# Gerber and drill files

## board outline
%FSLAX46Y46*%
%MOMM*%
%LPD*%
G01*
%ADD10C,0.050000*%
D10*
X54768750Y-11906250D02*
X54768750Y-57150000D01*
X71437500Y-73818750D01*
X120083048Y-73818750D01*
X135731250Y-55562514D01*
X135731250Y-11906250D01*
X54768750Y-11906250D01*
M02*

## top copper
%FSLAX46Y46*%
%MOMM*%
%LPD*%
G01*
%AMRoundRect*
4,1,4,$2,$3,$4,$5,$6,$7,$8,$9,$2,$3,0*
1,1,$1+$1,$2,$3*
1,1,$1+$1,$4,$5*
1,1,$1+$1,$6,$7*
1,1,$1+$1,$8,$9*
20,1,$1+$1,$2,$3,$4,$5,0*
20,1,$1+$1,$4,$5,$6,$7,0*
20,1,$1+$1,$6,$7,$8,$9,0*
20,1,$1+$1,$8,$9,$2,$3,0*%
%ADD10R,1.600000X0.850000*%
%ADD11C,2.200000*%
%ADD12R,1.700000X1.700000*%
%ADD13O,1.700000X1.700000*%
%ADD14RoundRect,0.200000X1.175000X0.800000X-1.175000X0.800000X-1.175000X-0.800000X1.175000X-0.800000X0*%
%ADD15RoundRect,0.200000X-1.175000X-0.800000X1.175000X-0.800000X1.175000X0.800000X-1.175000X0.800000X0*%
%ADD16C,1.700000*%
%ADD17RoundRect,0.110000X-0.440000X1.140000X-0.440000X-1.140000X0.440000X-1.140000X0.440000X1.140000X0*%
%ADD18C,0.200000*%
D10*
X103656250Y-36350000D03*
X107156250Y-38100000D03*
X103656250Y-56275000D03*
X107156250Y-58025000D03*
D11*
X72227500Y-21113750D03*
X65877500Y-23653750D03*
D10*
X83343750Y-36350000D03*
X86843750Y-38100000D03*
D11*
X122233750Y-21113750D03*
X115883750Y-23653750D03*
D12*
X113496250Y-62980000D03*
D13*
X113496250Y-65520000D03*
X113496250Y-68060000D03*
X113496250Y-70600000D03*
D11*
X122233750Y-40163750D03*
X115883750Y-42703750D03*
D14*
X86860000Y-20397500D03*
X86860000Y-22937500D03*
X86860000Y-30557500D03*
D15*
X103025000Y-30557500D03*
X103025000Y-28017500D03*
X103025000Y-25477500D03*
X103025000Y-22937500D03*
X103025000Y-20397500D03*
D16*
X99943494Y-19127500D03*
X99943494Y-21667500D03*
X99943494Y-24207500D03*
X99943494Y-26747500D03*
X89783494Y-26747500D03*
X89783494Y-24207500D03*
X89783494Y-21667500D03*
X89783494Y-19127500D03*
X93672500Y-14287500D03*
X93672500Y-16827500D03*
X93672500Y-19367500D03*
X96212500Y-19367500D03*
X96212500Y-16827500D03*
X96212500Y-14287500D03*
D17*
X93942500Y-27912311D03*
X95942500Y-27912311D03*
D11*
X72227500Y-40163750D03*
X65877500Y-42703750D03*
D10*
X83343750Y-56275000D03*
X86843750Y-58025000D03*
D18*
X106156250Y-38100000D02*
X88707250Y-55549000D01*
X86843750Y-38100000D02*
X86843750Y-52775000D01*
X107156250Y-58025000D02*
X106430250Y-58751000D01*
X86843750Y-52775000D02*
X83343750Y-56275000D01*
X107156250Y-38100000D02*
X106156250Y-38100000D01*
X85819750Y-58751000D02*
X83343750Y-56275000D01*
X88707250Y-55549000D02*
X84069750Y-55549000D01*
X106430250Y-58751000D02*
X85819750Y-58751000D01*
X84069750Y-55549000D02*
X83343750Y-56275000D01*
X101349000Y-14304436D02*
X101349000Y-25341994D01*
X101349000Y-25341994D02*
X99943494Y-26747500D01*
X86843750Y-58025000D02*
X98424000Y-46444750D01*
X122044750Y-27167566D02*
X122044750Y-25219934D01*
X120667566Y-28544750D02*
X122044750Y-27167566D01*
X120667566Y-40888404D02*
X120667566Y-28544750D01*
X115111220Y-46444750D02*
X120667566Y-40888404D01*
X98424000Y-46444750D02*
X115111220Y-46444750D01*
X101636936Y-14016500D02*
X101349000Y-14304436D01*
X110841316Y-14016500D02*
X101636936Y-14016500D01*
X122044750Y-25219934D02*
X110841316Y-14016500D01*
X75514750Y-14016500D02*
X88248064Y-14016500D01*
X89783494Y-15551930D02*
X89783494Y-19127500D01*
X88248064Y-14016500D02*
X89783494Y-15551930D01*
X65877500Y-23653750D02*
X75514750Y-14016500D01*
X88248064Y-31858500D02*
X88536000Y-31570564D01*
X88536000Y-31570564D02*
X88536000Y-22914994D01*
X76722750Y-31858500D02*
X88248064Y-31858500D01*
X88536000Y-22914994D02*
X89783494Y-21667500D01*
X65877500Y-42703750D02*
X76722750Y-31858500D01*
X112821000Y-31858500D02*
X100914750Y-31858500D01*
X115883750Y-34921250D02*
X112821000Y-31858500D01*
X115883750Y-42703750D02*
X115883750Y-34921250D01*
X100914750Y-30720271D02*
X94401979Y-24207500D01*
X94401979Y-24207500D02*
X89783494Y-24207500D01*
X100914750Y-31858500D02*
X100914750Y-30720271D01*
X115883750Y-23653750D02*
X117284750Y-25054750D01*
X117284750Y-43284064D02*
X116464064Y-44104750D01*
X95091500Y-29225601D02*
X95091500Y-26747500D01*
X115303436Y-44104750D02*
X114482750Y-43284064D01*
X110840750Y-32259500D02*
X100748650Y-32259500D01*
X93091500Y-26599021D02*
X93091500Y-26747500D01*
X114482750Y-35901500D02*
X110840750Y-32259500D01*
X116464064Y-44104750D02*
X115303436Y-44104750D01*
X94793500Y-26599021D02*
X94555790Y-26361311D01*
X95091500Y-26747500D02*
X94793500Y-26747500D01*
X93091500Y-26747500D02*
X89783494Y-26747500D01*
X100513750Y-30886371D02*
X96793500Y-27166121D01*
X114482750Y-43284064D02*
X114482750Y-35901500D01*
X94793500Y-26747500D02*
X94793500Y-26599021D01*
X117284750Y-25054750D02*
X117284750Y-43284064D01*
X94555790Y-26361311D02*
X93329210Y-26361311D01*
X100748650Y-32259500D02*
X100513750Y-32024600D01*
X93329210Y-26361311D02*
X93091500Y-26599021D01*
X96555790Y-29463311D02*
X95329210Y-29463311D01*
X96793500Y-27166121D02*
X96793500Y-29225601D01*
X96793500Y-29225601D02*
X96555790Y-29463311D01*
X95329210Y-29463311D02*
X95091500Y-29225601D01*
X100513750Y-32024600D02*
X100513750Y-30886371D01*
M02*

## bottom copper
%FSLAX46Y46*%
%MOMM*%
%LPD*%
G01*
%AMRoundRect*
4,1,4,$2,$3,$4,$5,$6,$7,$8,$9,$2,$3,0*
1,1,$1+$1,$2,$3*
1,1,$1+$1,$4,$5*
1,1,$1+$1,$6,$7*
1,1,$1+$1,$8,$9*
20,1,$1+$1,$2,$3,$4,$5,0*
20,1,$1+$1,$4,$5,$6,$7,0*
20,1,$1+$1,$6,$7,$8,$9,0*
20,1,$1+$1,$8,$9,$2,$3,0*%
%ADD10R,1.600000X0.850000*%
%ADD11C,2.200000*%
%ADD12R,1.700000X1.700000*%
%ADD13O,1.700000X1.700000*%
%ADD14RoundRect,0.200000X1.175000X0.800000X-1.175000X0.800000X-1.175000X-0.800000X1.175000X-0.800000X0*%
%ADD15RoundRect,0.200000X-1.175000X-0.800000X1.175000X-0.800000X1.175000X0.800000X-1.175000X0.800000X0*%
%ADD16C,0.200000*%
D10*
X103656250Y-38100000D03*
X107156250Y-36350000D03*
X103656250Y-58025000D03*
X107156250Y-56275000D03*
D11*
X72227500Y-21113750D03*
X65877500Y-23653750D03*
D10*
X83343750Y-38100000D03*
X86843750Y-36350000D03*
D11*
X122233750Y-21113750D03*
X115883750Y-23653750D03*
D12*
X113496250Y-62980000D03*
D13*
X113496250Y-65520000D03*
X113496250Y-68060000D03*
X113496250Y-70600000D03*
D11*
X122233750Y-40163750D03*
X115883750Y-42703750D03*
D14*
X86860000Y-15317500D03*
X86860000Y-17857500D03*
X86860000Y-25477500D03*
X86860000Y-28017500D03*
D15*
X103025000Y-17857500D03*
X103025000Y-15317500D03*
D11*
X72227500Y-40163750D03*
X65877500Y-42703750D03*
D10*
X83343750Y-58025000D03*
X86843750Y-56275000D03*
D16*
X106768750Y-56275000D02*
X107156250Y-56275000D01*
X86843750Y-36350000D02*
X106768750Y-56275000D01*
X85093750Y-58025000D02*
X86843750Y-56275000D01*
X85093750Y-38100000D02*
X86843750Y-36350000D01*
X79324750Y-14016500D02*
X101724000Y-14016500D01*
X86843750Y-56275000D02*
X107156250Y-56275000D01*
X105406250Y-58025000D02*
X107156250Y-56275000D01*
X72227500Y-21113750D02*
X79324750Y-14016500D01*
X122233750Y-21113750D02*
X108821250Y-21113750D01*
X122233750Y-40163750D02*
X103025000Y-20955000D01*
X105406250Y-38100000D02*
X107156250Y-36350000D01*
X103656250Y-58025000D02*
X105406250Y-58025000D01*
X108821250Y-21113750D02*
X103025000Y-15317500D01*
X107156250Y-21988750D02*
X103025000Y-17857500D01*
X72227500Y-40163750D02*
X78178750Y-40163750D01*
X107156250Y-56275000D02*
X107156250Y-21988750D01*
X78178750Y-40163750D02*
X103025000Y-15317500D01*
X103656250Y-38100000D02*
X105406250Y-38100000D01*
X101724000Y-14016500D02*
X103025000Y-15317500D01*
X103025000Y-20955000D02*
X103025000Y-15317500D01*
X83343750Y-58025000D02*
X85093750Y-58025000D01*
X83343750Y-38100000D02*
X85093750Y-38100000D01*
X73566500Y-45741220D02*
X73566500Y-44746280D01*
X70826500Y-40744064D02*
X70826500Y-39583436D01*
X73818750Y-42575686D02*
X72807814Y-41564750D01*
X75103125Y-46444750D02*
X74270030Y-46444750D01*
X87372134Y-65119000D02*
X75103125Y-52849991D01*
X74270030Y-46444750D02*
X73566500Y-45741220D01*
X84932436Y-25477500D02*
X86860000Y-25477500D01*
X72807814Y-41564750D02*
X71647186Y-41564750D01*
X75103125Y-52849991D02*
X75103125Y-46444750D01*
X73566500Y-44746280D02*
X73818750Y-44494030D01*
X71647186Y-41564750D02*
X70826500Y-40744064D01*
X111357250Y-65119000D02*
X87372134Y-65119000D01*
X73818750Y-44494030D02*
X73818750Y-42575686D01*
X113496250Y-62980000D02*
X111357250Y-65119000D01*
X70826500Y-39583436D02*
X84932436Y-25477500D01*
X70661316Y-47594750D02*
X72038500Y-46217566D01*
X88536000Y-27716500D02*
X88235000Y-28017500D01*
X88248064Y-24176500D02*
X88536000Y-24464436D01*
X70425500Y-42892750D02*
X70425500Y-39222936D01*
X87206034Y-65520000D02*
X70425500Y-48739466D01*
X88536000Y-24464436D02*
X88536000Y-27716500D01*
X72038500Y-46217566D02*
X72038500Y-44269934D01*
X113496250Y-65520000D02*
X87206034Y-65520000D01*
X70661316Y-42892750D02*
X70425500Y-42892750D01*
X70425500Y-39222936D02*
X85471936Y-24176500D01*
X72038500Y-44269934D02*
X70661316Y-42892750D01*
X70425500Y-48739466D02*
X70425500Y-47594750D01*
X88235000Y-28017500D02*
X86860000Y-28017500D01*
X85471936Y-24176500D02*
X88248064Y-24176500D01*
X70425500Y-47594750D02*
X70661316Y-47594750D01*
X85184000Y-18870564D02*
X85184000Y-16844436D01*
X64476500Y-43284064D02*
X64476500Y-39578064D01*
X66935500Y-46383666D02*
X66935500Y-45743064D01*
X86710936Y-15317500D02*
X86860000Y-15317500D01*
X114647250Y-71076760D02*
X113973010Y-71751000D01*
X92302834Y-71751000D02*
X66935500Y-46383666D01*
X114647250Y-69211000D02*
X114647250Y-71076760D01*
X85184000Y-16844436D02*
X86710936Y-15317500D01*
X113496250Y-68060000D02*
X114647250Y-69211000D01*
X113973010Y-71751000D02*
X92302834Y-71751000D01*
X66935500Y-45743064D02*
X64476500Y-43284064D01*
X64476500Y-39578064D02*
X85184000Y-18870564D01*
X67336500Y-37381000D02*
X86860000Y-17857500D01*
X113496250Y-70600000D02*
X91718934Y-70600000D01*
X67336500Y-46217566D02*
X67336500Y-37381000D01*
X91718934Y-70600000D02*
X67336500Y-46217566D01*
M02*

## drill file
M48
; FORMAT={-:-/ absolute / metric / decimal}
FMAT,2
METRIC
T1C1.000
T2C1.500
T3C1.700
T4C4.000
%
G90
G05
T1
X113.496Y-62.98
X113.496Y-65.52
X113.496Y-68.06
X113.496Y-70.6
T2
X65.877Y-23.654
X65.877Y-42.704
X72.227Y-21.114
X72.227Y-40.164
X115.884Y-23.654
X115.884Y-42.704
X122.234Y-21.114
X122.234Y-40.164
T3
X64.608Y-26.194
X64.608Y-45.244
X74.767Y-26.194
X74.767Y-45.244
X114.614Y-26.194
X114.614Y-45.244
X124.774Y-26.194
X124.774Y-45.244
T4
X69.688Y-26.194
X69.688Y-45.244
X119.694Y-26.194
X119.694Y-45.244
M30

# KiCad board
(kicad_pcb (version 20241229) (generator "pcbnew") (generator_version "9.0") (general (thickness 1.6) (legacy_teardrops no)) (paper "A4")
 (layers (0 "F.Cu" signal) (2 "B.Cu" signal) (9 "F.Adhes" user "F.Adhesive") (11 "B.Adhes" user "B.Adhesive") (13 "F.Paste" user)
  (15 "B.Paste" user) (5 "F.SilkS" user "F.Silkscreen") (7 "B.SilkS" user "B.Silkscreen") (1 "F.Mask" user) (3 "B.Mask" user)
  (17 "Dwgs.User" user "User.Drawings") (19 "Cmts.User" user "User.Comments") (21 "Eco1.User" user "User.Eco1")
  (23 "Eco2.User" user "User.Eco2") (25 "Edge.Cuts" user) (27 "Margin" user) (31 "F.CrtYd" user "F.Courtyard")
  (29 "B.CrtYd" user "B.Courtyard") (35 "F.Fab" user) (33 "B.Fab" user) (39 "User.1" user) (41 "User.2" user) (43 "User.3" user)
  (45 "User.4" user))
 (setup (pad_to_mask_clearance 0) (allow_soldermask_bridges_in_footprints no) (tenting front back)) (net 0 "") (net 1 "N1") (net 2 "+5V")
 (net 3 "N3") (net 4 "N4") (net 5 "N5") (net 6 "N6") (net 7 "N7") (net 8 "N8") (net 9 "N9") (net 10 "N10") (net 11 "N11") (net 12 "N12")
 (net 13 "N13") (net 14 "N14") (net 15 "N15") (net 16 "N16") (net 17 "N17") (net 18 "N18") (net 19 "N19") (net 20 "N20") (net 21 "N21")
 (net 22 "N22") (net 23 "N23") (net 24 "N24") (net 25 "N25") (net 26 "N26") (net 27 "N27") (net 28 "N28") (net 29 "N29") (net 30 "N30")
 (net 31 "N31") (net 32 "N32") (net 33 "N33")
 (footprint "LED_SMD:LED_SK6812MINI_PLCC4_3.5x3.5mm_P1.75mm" (layer "F.Cu") (at 105.40625 37.225)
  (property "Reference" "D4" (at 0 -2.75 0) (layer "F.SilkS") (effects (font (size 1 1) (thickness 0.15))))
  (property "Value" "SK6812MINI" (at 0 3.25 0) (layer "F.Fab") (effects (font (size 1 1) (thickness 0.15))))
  (pad "1" smd rect (at -1.75 -0.875) (size 1.6 0.85) (layers "F.Cu" "F.Mask" "F.Paste") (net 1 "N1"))
  (pad "2" smd rect (at -1.75 0.875) (size 1.6 0.85) (layers "F.Mask" "B.Cu" "F.Paste") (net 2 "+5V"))
  (pad "3" smd rect (at 1.75 0.875) (size 1.6 0.85) (layers "F.Cu" "F.Mask" "F.Paste") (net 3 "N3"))
  (pad "4" smd rect (at 1.75 -0.875) (size 1.6 0.85) (layers "F.Mask" "B.Cu" "F.Paste") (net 2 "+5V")))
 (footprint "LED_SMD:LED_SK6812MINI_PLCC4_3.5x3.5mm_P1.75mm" (layer "F.Cu") (at 105.40625 57.15)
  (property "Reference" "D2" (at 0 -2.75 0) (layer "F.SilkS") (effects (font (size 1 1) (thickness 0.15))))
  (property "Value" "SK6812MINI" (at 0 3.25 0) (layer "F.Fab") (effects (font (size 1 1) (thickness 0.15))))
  (pad "1" smd rect (at -1.75 -0.875) (size 1.6 0.85) (layers "F.Cu" "F.Mask" "F.Paste") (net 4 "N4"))
  (pad "2" smd rect (at -1.75 0.875) (size 1.6 0.85) (layers "F.Mask" "B.Cu" "F.Paste") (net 2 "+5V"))
  (pad "3" smd rect (at 1.75 0.875) (size 1.6 0.85) (layers "F.Cu" "F.Mask" "F.Paste") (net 3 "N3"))
  (pad "4" smd rect (at 1.75 -0.875) (size 1.6 0.85) (layers "F.Mask" "B.Cu" "F.Paste") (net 2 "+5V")))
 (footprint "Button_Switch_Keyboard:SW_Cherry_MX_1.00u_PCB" (layer "F.Cu") (at 72.2275 21.11375)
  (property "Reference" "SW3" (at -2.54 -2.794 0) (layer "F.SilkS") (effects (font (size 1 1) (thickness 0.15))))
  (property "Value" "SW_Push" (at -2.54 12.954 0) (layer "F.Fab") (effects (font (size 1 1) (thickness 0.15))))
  (pad "" np_thru_hole circle (at -7.62 5.08) (size 1.7 1.7) (drill 1.7) (layers "*.Cu" "*.Mask"))
  (pad "" np_thru_hole circle (at -2.54 5.08) (size 4 4) (drill 4) (layers "*.Cu" "*.Mask"))
  (pad "" np_thru_hole circle (at 2.54 5.08) (size 1.7 1.7) (drill 1.7) (layers "*.Cu" "*.Mask"))
  (pad "1" thru_hole circle (at 0 0) (size 2.2 2.2) (drill 1.5) (layers "*.Cu" "*.Mask") (remove_unused_layers no) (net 2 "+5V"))
  (pad "2" thru_hole circle (at -6.35 2.54) (size 2.2 2.2) (drill 1.5) (layers "*.Cu" "*.Mask") (remove_unused_layers no) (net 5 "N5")))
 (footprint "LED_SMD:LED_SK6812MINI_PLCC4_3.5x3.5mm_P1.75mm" (layer "F.Cu") (at 85.09375 37.225)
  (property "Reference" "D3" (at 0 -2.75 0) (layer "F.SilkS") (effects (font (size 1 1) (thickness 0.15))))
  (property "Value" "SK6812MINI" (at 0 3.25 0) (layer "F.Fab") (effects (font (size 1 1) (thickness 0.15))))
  (pad "1" smd rect (at -1.75 -0.875) (size 1.6 0.85) (layers "F.Cu" "F.Mask" "F.Paste") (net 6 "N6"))
  (pad "2" smd rect (at -1.75 0.875) (size 1.6 0.85) (layers "F.Mask" "B.Cu" "F.Paste") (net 2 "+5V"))
  (pad "3" smd rect (at 1.75 0.875) (size 1.6 0.85) (layers "F.Cu" "F.Mask" "F.Paste") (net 3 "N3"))
  (pad "4" smd rect (at 1.75 -0.875) (size 1.6 0.85) (layers "F.Mask" "B.Cu" "F.Paste") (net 2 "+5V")))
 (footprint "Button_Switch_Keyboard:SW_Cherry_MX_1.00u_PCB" (layer "F.Cu") (at 122.23375 21.11375)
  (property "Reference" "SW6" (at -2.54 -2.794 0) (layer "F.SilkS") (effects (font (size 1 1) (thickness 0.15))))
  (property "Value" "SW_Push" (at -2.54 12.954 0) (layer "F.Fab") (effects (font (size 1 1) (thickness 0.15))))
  (pad "" np_thru_hole circle (at -7.62 5.08) (size 1.7 1.7) (drill 1.7) (layers "*.Cu" "*.Mask"))
  (pad "" np_thru_hole circle (at -2.54 5.08) (size 4 4) (drill 4) (layers "*.Cu" "*.Mask"))
  (pad "" np_thru_hole circle (at 2.54 5.08) (size 1.7 1.7) (drill 1.7) (layers "*.Cu" "*.Mask"))
  (pad "1" thru_hole circle (at 0 0) (size 2.2 2.2) (drill 1.5) (layers "*.Cu" "*.Mask") (remove_unused_layers no) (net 2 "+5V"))
  (pad "2" thru_hole circle (at -6.35 2.54) (size 2.2 2.2) (drill 1.5) (layers "*.Cu" "*.Mask") (remove_unused_layers no) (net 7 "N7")))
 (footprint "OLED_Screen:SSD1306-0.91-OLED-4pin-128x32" (layer "F.Cu") (at 76.99625 60.79)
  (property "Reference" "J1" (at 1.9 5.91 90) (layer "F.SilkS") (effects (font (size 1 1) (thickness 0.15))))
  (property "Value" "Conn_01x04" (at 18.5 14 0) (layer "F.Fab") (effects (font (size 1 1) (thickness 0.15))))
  (pad "1" thru_hole rect (at 36.5 2.19) (size 1.7 1.7) (drill 1) (layers "*.Cu" "*.Mask") (remove_unused_layers no) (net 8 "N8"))
  (pad "2" thru_hole oval (at 36.5 4.73) (size 1.7 1.7) (drill 1) (layers "*.Cu" "*.Mask") (remove_unused_layers no) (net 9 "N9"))
  (pad "3" thru_hole oval (at 36.5 7.27) (size 1.7 1.7) (drill 1) (layers "*.Cu" "*.Mask") (remove_unused_layers no) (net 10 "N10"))
  (pad "4" thru_hole oval (at 36.5 9.81) (size 1.7 1.7) (drill 1) (layers "*.Cu" "*.Mask") (remove_unused_layers no) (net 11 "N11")))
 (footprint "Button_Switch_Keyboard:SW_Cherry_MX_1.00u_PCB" (layer "F.Cu") (at 122.23375 40.16375)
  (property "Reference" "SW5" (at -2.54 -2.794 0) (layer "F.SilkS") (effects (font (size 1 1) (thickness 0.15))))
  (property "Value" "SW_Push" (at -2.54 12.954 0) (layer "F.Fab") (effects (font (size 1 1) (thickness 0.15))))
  (pad "" np_thru_hole circle (at -7.62 5.08) (size 1.7 1.7) (drill 1.7) (layers "*.Cu" "*.Mask"))
  (pad "" np_thru_hole circle (at -2.54 5.08) (size 4 4) (drill 4) (layers "*.Cu" "*.Mask"))
  (pad "" np_thru_hole circle (at 2.54 5.08) (size 1.7 1.7) (drill 1.7) (layers "*.Cu" "*.Mask"))
  (pad "1" thru_hole circle (at 0 0) (size 2.2 2.2) (drill 1.5) (layers "*.Cu" "*.Mask") (remove_unused_layers no) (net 2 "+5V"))
  (pad "2" thru_hole circle (at -6.35 2.54) (size 2.2 2.2) (drill 1.5) (layers "*.Cu" "*.Mask") (remove_unused_layers no) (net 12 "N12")))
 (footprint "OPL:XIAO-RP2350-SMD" (layer "F.Cu") (at 94.86 22.9375)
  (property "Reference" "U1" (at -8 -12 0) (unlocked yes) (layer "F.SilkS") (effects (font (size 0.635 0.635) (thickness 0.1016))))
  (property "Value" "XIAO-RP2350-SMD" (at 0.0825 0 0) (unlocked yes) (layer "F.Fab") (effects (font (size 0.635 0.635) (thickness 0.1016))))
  (pad "1" smd roundrect (at -8 -7.62 180) (size 2.75 2) (layers "F.Mask" "B.Cu" "F.Paste") (roundrect_rratio 0.1) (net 10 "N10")
   (thermal_bridge_angle 45))
  (pad "2" smd roundrect (at -8 -5.08 180) (size 2.75 2) (layers "F.Mask" "B.Cu" "F.Paste") (roundrect_rratio 0.1) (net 11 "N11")
   (thermal_bridge_angle 45))
  (pad "3" smd roundrect (at -8 -2.54 180) (size 2.75 2) (layers "F.Cu" "F.Mask" "F.Paste") (roundrect_rratio 0.1) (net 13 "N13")
   (thermal_bridge_angle 45))
  (pad "4" smd roundrect (at -8 0 180) (size 2.75 2) (layers "F.Cu" "F.Mask" "F.Paste") (roundrect_rratio 0.1) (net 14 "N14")
   (thermal_bridge_angle 45))
  (pad "5" smd roundrect (at -8 2.54 180) (size 2.75 2) (layers "F.Mask" "B.Cu" "F.Paste") (roundrect_rratio 0.1) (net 8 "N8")
   (thermal_bridge_angle 45))
  (pad "6" smd roundrect (at -8 5.08 180) (size 2.75 2) (layers "F.Mask" "B.Cu" "F.Paste") (roundrect_rratio 0.1) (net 9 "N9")
   (thermal_bridge_angle 45))
  (pad "7" smd roundrect (at -8 7.62 180) (size 2.75 2) (layers "F.Cu" "F.Mask" "F.Paste") (roundrect_rratio 0.1) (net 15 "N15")
   (thermal_bridge_angle 45))
  (pad "8" smd roundrect (at 8.165 7.62) (size 2.75 2) (layers "F.Cu" "F.Mask" "F.Paste") (roundrect_rratio 0.1) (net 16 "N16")
   (thermal_bridge_angle 45))
  (pad "9" smd roundrect (at 8.165 5.08) (size 2.75 2) (layers "F.Cu" "F.Mask" "F.Paste") (roundrect_rratio 0.1) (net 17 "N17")
   (thermal_bridge_angle 45))
  (pad "10" smd roundrect (at 8.165 2.54) (size 2.75 2) (layers "F.Cu" "F.Mask" "F.Paste") (roundrect_rratio 0.1) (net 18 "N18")
   (thermal_bridge_angle 45))
  (pad "11" smd roundrect (at 8.165 0) (size 2.75 2) (layers "F.Cu" "F.Mask" "F.Paste") (roundrect_rratio 0.1) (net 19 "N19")
   (thermal_bridge_angle 45))
  (pad "12" smd roundrect (at 8.165 -2.54) (size 2.75 2) (layers "F.Cu" "F.Mask" "F.Paste") (roundrect_rratio 0.1) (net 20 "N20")
   (thermal_bridge_angle 45))
  (pad "13" smd roundrect (at 8.165 -5.08) (size 2.75 2) (layers "F.Mask" "B.Cu" "F.Paste") (roundrect_rratio 0.1) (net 2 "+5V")
   (thermal_bridge_angle 45))
  (pad "14" smd roundrect (at 8.165 -7.62) (size 2.75 2) (layers "F.Mask" "B.Cu" "F.Paste") (roundrect_rratio 0.1) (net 2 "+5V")
   (thermal_bridge_angle 45))
  (pad "15" smd circle (at 5.083494 -3.81 180) (size 1.7 1.7) (layers "F.Cu" "F.Mask" "F.Paste") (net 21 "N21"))
  (pad "16" smd circle (at 5.083494 -1.27 180) (size 1.7 1.7) (layers "F.Cu" "F.Mask" "F.Paste") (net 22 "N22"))
  (pad "17" smd circle (at 5.083494 1.27 180) (size 1.7 1.7) (layers "F.Cu" "F.Mask" "F.Paste") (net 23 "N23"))
  (pad "18" smd circle (at 5.083494 3.81 180) (size 1.7 1.7) (layers "F.Cu" "F.Mask" "F.Paste") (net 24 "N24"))
  (pad "19" smd circle (at -5.076506 3.81 180) (size 1.7 1.7) (layers "F.Cu" "F.Mask" "F.Paste") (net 7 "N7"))
  (pad "20" smd circle (at -5.076506 1.27 180) (size 1.7 1.7) (layers "F.Cu" "F.Mask" "F.Paste") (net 12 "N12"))
  (pad "21" smd circle (at -5.076506 -1.27 180) (size 1.7 1.7) (layers "F.Cu" "F.Mask" "F.Paste") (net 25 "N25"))
  (pad "22" smd circle (at -5.076506 -3.81 180) (size 1.7 1.7) (layers "F.Cu" "F.Mask" "F.Paste") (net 5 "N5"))
  (pad "23" smd circle (at -1.1875 -8.65 180) (size 1.7 1.7) (layers "F.Cu" "F.Mask" "F.Paste") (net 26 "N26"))
  (pad "24" smd circle (at -1.1875 -6.11 180) (size 1.7 1.7) (layers "F.Cu" "F.Mask" "F.Paste") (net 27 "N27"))
  (pad "25" smd circle (at -1.1875 -3.57 180) (size 1.7 1.7) (layers "F.Cu" "F.Mask" "F.Paste") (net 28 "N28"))
  (pad "26" smd circle (at 1.3525 -3.57 180) (size 1.7 1.7) (layers "F.Cu" "F.Mask" "F.Paste") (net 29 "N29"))
  (pad "27" smd circle (at 1.3525 -6.11 180) (size 1.7 1.7) (layers "F.Cu" "F.Mask" "F.Paste") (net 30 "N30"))
  (pad "28" smd circle (at 1.3525 -8.65 180) (size 1.7 1.7) (layers "F.Cu" "F.Mask" "F.Paste") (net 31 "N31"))
  (pad "29" smd roundrect (at -0.9175 4.974811 270) (size 2.5 1.1) (layers "F.Cu" "F.Mask" "F.Paste") (roundrect_rratio 0.1) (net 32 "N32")
   (thermal_bridge_angle 45))
  (pad "30" smd roundrect (at 1.0825 4.974811 270) (size 2.5 1.1) (layers "F.Cu" "F.Mask" "F.Paste") (roundrect_rratio 0.1) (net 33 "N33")
   (thermal_bridge_angle 45)))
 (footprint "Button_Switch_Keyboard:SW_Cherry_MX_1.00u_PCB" (layer "F.Cu") (at 72.2275 40.16375)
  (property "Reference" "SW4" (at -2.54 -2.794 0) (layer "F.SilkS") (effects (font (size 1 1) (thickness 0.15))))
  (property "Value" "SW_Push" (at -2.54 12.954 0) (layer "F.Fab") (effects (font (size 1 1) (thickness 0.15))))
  (pad "" np_thru_hole circle (at -7.62 5.08) (size 1.7 1.7) (drill 1.7) (layers "*.Cu" "*.Mask"))
  (pad "" np_thru_hole circle (at -2.54 5.08) (size 4 4) (drill 4) (layers "*.Cu" "*.Mask"))
  (pad "" np_thru_hole circle (at 2.54 5.08) (size 1.7 1.7) (drill 1.7) (layers "*.Cu" "*.Mask"))
  (pad "1" thru_hole circle (at 0 0) (size 2.2 2.2) (drill 1.5) (layers "*.Cu" "*.Mask") (remove_unused_layers no) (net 2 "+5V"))
  (pad "2" thru_hole circle (at -6.35 2.54) (size 2.2 2.2) (drill 1.5) (layers "*.Cu" "*.Mask") (remove_unused_layers no) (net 25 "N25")))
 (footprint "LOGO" (layer "F.Cu") (at 95.25 47.625)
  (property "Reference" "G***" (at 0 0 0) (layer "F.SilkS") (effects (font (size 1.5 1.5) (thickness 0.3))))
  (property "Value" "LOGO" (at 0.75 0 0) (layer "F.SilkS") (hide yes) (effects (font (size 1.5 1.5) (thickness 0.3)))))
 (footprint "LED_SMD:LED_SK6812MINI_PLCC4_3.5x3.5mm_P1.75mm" (layer "F.Cu") (at 85.09375 57.15)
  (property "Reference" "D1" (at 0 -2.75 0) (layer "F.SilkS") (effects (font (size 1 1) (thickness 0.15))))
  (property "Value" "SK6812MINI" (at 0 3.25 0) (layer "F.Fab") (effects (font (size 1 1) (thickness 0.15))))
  (pad "1" smd rect (at -1.75 -0.875) (size 1.6 0.85) (layers "F.Cu" "F.Mask" "F.Paste") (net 3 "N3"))
  (pad "2" smd rect (at -1.75 0.875) (size 1.6 0.85) (layers "F.Mask" "B.Cu" "F.Paste") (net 2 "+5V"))
  (pad "3" smd rect (at 1.75 0.875) (size 1.6 0.85) (layers "F.Cu" "F.Mask" "F.Paste") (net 24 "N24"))
  (pad "4" smd rect (at 1.75 -0.875) (size 1.6 0.85) (layers "F.Mask" "B.Cu" "F.Paste") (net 2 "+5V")))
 (gr_poly
  (pts (xy 54.76875 11.90625) (xy 54.76875 57.15) (xy 71.4375 73.81875) (xy 120.083048 73.81875) (xy 135.73125 55.562514)
   (xy 135.73125 11.90625))
  (stroke (width 0.05) (type solid)) (fill no) (layer "Edge.Cuts"))
 (segment (start 106.76875 56.275) (end 107.15625 56.275) (width 0.2) (layer "B.Cu") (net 2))
 (segment (start 86.84375 36.35) (end 106.76875 56.275) (width 0.2) (layer "B.Cu") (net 2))
 (segment (start 85.09375 58.025) (end 86.84375 56.275) (width 0.2) (layer "B.Cu") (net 2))
 (segment (start 85.09375 38.1) (end 86.84375 36.35) (width 0.2) (layer "B.Cu") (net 2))
 (segment (start 79.32475 14.0165) (end 101.724 14.0165) (width 0.2) (layer "B.Cu") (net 2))
 (segment (start 86.84375 56.275) (end 107.15625 56.275) (width 0.2) (layer "B.Cu") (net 2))
 (segment (start 105.40625 58.025) (end 107.15625 56.275) (width 0.2) (layer "B.Cu") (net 2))
 (segment (start 72.2275 21.11375) (end 79.32475 14.0165) (width 0.2) (layer "B.Cu") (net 2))
 (segment (start 122.23375 21.11375) (end 108.82125 21.11375) (width 0.2) (layer "B.Cu") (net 2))
 (segment (start 122.23375 40.16375) (end 103.025 20.955) (width 0.2) (layer "B.Cu") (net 2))
 (segment (start 105.40625 38.1) (end 107.15625 36.35) (width 0.2) (layer "B.Cu") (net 2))
 (segment (start 103.65625 58.025) (end 105.40625 58.025) (width 0.2) (layer "B.Cu") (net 2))
 (segment (start 108.82125 21.11375) (end 103.025 15.3175) (width 0.2) (layer "B.Cu") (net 2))
 (segment (start 107.15625 21.98875) (end 103.025 17.8575) (width 0.2) (layer "B.Cu") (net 2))
 (segment (start 72.2275 40.16375) (end 78.17875 40.16375) (width 0.2) (layer "B.Cu") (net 2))
 (segment (start 107.15625 56.275) (end 107.15625 21.98875) (width 0.2) (layer "B.Cu") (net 2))
 (segment (start 78.17875 40.16375) (end 103.025 15.3175) (width 0.2) (layer "B.Cu") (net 2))
 (segment (start 103.65625 38.1) (end 105.40625 38.1) (width 0.2) (layer "B.Cu") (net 2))
 (segment (start 101.724 14.0165) (end 103.025 15.3175) (width 0.2) (layer "B.Cu") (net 2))
 (segment (start 103.025 20.955) (end 103.025 15.3175) (width 0.2) (layer "B.Cu") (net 2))
 (segment (start 83.34375 58.025) (end 85.09375 58.025) (width 0.2) (layer "B.Cu") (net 2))
 (segment (start 83.34375 38.1) (end 85.09375 38.1) (width 0.2) (layer "B.Cu") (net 2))
 (segment (start 106.15625 38.1) (end 88.70725 55.549) (width 0.2) (layer "F.Cu") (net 3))
 (segment (start 86.84375 38.1) (end 86.84375 52.775) (width 0.2) (layer "F.Cu") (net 3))
 (segment (start 107.15625 58.025) (end 106.43025 58.751) (width 0.2) (layer "F.Cu") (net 3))
 (segment (start 86.84375 52.775) (end 83.34375 56.275) (width 0.2) (layer "F.Cu") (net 3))
 (segment (start 107.15625 38.1) (end 106.15625 38.1) (width 0.2) (layer "F.Cu") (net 3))
 (segment (start 85.81975 58.751) (end 83.34375 56.275) (width 0.2) (layer "F.Cu") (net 3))
 (segment (start 88.70725 55.549) (end 84.06975 55.549) (width 0.2) (layer "F.Cu") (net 3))
 (segment (start 106.43025 58.751) (end 85.81975 58.751) (width 0.2) (layer "F.Cu") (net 3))
 (segment (start 84.06975 55.549) (end 83.34375 56.275) (width 0.2) (layer "F.Cu") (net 3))
 (segment (start 101.349 14.304436) (end 101.349 25.341994) (width 0.2) (layer "F.Cu") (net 24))
 (segment (start 101.349 25.341994) (end 99.943494 26.7475) (width 0.2) (layer "F.Cu") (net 24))
 (segment (start 86.84375 58.025) (end 98.424 46.44475) (width 0.2) (layer "F.Cu") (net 24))
 (segment (start 122.04475 27.167566) (end 122.04475 25.219934) (width 0.2) (layer "F.Cu") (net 24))
 (segment (start 120.667566 28.54475) (end 122.04475 27.167566) (width 0.2) (layer "F.Cu") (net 24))
 (segment (start 120.667566 40.888404) (end 120.667566 28.54475) (width 0.2) (layer "F.Cu") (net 24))
 (segment (start 115.11122 46.44475) (end 120.667566 40.888404) (width 0.2) (layer "F.Cu") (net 24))
 (segment (start 98.424 46.44475) (end 115.11122 46.44475) (width 0.2) (layer "F.Cu") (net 24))
 (segment (start 101.636936 14.0165) (end 101.349 14.304436) (width 0.2) (layer "F.Cu") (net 24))
 (segment (start 110.841316 14.0165) (end 101.636936 14.0165) (width 0.2) (layer "F.Cu") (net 24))
 (segment (start 122.04475 25.219934) (end 110.841316 14.0165) (width 0.2) (layer "F.Cu") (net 24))
 (segment (start 73.5665 45.74122) (end 73.5665 44.74628) (width 0.2) (layer "B.Cu") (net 8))
 (segment (start 70.8265 40.744064) (end 70.8265 39.583436) (width 0.2) (layer "B.Cu") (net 8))
 (segment (start 73.81875 42.575686) (end 72.807814 41.56475) (width 0.2) (layer "B.Cu") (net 8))
 (segment (start 75.103125 46.44475) (end 74.27003 46.44475) (width 0.2) (layer "B.Cu") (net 8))
 (segment (start 87.372134 65.119) (end 75.103125 52.849991) (width 0.2) (layer "B.Cu") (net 8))
 (segment (start 74.27003 46.44475) (end 73.5665 45.74122) (width 0.2) (layer "B.Cu") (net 8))
 (segment (start 84.932436 25.4775) (end 86.86 25.4775) (width 0.2) (layer "B.Cu") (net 8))
 (segment (start 72.807814 41.56475) (end 71.647186 41.56475) (width 0.2) (layer "B.Cu") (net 8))
 (segment (start 75.103125 52.849991) (end 75.103125 46.44475) (width 0.2) (layer "B.Cu") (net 8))
 (segment (start 73.5665 44.74628) (end 73.81875 44.49403) (width 0.2) (layer "B.Cu") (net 8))
 (segment (start 71.647186 41.56475) (end 70.8265 40.744064) (width 0.2) (layer "B.Cu") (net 8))
 (segment (start 111.35725 65.119) (end 87.372134 65.119) (width 0.2) (layer "B.Cu") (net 8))
 (segment (start 73.81875 44.49403) (end 73.81875 42.575686) (width 0.2) (layer "B.Cu") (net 8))
 (segment (start 113.49625 62.98) (end 111.35725 65.119) (width 0.2) (layer "B.Cu") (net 8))
 (segment (start 70.8265 39.583436) (end 84.932436 25.4775) (width 0.2) (layer "B.Cu") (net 8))
 (segment (start 70.661316 47.59475) (end 72.0385 46.217566) (width 0.2) (layer "B.Cu") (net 9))
 (segment (start 88.536 27.7165) (end 88.235 28.0175) (width 0.2) (layer "B.Cu") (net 9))
 (segment (start 88.248064 24.1765) (end 88.536 24.464436) (width 0.2) (layer "B.Cu") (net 9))
 (segment (start 70.4255 42.89275) (end 70.4255 39.222936) (width 0.2) (layer "B.Cu") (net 9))
 (segment (start 87.206034 65.52) (end 70.4255 48.739466) (width 0.2) (layer "B.Cu") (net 9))
 (segment (start 88.536 24.464436) (end 88.536 27.7165) (width 0.2) (layer "B.Cu") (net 9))
 (segment (start 72.0385 46.217566) (end 72.0385 44.269934) (width 0.2) (layer "B.Cu") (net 9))
 (segment (start 113.49625 65.52) (end 87.206034 65.52) (width 0.2) (layer "B.Cu") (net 9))
 (segment (start 70.661316 42.89275) (end 70.4255 42.89275) (width 0.2) (layer "B.Cu") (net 9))
 (segment (start 70.4255 39.222936) (end 85.471936 24.1765) (width 0.2) (layer "B.Cu") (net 9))
 (segment (start 72.0385 44.269934) (end 70.661316 42.89275) (width 0.2) (layer "B.Cu") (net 9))
 (segment (start 70.4255 48.739466) (end 70.4255 47.59475) (width 0.2) (layer "B.Cu") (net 9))
 (segment (start 88.235 28.0175) (end 86.86 28.0175) (width 0.2) (layer "B.Cu") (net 9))
 (segment (start 85.471936 24.1765) (end 88.248064 24.1765) (width 0.2) (layer "B.Cu") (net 9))
 (segment (start 70.4255 47.59475) (end 70.661316 47.59475) (width 0.2) (layer "B.Cu") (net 9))
 (segment (start 85.184 18.870564) (end 85.184 16.844436) (width 0.2) (layer "B.Cu") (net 10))
 (segment (start 64.4765 43.284064) (end 64.4765 39.578064) (width 0.2) (layer "B.Cu") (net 10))
 (segment (start 66.9355 46.383666) (end 66.9355 45.743064) (width 0.2) (layer "B.Cu") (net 10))
 (segment (start 86.710936 15.3175) (end 86.86 15.3175) (width 0.2) (layer "B.Cu") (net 10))
 (segment (start 114.64725 71.07676) (end 113.97301 71.751) (width 0.2) (layer "B.Cu") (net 10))
 (segment (start 92.302834 71.751) (end 66.9355 46.383666) (width 0.2) (layer "B.Cu") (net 10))
 (segment (start 114.64725 69.211) (end 114.64725 71.07676) (width 0.2) (layer "B.Cu") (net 10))
 (segment (start 85.184 16.844436) (end 86.710936 15.3175) (width 0.2) (layer "B.Cu") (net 10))
 (segment (start 113.49625 68.06) (end 114.64725 69.211) (width 0.2) (layer "B.Cu") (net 10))
 (segment (start 113.97301 71.751) (end 92.302834 71.751) (width 0.2) (layer "B.Cu") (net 10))
 (segment (start 66.9355 45.743064) (end 64.4765 43.284064) (width 0.2) (layer "B.Cu") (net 10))
 (segment (start 64.4765 39.578064) (end 85.184 18.870564) (width 0.2) (layer "B.Cu") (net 10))
 (segment (start 67.3365 37.381) (end 86.86 17.8575) (width 0.2) (layer "B.Cu") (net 11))
 (segment (start 113.49625 70.6) (end 91.718934 70.6) (width 0.2) (layer "B.Cu") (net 11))
 (segment (start 67.3365 46.217566) (end 67.3365 37.381) (width 0.2) (layer "B.Cu") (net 11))
 (segment (start 91.718934 70.6) (end 67.3365 46.217566) (width 0.2) (layer "B.Cu") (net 11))
 (segment (start 75.51475 14.0165) (end 88.248064 14.0165) (width 0.2) (layer "F.Cu") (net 5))
 (segment (start 89.783494 15.55193) (end 89.783494 19.1275) (width 0.2) (layer "F.Cu") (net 5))
 (segment (start 88.248064 14.0165) (end 89.783494 15.55193) (width 0.2) (layer "F.Cu") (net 5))
 (segment (start 65.8775 23.65375) (end 75.51475 14.0165) (width 0.2) (layer "F.Cu") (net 5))
 (segment (start 88.248064 31.8585) (end 88.536 31.570564) (width 0.2) (layer "F.Cu") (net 25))
 (segment (start 88.536 31.570564) (end 88.536 22.914994) (width 0.2) (layer "F.Cu") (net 25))
 (segment (start 76.72275 31.8585) (end 88.248064 31.8585) (width 0.2) (layer "F.Cu") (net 25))
 (segment (start 88.536 22.914994) (end 89.783494 21.6675) (width 0.2) (layer "F.Cu") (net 25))
 (segment (start 65.8775 42.70375) (end 76.72275 31.8585) (width 0.2) (layer "F.Cu") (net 25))
 (segment (start 112.821 31.8585) (end 100.91475 31.8585) (width 0.2) (layer "F.Cu") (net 12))
 (segment (start 115.88375 34.92125) (end 112.821 31.8585) (width 0.2) (layer "F.Cu") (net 12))
 (segment (start 115.88375 42.70375) (end 115.88375 34.92125) (width 0.2) (layer "F.Cu") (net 12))
 (segment (start 100.91475 30.720271) (end 94.401979 24.2075) (width 0.2) (layer "F.Cu") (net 12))
 (segment (start 94.401979 24.2075) (end 89.783494 24.2075) (width 0.2) (layer "F.Cu") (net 12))
 (segment (start 100.91475 31.8585) (end 100.91475 30.720271) (width 0.2) (layer "F.Cu") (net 12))
 (segment (start 115.88375 23.65375) (end 117.28475 25.05475) (width 0.2) (layer "F.Cu") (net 7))
 (segment (start 117.28475 43.284064) (end 116.464064 44.10475) (width 0.2) (layer "F.Cu") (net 7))
 (segment (start 95.0915 29.225601) (end 95.0915 26.7475) (width 0.2) (layer "F.Cu") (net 7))
 (segment (start 115.303436 44.10475) (end 114.48275 43.284064) (width 0.2) (layer "F.Cu") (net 7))
 (segment (start 110.84075 32.2595) (end 100.74865 32.2595) (width 0.2) (layer "F.Cu") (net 7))
 (segment (start 93.0915 26.599021) (end 93.0915 26.7475) (width 0.2) (layer "F.Cu") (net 7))
 (segment (start 114.48275 35.9015) (end 110.84075 32.2595) (width 0.2) (layer "F.Cu") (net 7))
 (segment (start 116.464064 44.10475) (end 115.303436 44.10475) (width 0.2) (layer "F.Cu") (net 7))
 (segment (start 94.7935 26.599021) (end 94.55579 26.361311) (width 0.2) (layer "F.Cu") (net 7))
 (segment (start 95.0915 26.7475) (end 94.7935 26.7475) (width 0.2) (layer "F.Cu") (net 7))
 (segment (start 93.0915 26.7475) (end 89.783494 26.7475) (width 0.2) (layer "F.Cu") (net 7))
 (segment (start 100.51375 30.886371) (end 96.7935 27.166121) (width 0.2) (layer "F.Cu") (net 7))
 (segment (start 114.48275 43.284064) (end 114.48275 35.9015) (width 0.2) (layer "F.Cu") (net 7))
 (segment (start 94.7935 26.7475) (end 94.7935 26.599021) (width 0.2) (layer "F.Cu") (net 7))
 (segment (start 117.28475 25.05475) (end 117.28475 43.284064) (width 0.2) (layer "F.Cu") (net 7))
 (segment (start 94.55579 26.361311) (end 93.32921 26.361311) (width 0.2) (layer "F.Cu") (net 7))
 (segment (start 100.74865 32.2595) (end 100.51375 32.0246) (width 0.2) (layer "F.Cu") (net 7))
 (segment (start 93.32921 26.361311) (end 93.0915 26.599021) (width 0.2) (layer "F.Cu") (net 7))
 (segment (start 96.55579 29.463311) (end 95.32921 29.463311) (width 0.2) (layer "F.Cu") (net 7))
 (segment (start 96.7935 27.166121) (end 96.7935 29.225601) (width 0.2) (layer "F.Cu") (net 7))
 (segment (start 96.7935 29.225601) (end 96.55579 29.463311) (width 0.2) (layer "F.Cu") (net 7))
 (segment (start 95.32921 29.463311) (end 95.0915 29.225601) (width 0.2) (layer "F.Cu") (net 7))
 (segment (start 100.51375 32.0246) (end 100.51375 30.886371) (width 0.2) (layer "F.Cu") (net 7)))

